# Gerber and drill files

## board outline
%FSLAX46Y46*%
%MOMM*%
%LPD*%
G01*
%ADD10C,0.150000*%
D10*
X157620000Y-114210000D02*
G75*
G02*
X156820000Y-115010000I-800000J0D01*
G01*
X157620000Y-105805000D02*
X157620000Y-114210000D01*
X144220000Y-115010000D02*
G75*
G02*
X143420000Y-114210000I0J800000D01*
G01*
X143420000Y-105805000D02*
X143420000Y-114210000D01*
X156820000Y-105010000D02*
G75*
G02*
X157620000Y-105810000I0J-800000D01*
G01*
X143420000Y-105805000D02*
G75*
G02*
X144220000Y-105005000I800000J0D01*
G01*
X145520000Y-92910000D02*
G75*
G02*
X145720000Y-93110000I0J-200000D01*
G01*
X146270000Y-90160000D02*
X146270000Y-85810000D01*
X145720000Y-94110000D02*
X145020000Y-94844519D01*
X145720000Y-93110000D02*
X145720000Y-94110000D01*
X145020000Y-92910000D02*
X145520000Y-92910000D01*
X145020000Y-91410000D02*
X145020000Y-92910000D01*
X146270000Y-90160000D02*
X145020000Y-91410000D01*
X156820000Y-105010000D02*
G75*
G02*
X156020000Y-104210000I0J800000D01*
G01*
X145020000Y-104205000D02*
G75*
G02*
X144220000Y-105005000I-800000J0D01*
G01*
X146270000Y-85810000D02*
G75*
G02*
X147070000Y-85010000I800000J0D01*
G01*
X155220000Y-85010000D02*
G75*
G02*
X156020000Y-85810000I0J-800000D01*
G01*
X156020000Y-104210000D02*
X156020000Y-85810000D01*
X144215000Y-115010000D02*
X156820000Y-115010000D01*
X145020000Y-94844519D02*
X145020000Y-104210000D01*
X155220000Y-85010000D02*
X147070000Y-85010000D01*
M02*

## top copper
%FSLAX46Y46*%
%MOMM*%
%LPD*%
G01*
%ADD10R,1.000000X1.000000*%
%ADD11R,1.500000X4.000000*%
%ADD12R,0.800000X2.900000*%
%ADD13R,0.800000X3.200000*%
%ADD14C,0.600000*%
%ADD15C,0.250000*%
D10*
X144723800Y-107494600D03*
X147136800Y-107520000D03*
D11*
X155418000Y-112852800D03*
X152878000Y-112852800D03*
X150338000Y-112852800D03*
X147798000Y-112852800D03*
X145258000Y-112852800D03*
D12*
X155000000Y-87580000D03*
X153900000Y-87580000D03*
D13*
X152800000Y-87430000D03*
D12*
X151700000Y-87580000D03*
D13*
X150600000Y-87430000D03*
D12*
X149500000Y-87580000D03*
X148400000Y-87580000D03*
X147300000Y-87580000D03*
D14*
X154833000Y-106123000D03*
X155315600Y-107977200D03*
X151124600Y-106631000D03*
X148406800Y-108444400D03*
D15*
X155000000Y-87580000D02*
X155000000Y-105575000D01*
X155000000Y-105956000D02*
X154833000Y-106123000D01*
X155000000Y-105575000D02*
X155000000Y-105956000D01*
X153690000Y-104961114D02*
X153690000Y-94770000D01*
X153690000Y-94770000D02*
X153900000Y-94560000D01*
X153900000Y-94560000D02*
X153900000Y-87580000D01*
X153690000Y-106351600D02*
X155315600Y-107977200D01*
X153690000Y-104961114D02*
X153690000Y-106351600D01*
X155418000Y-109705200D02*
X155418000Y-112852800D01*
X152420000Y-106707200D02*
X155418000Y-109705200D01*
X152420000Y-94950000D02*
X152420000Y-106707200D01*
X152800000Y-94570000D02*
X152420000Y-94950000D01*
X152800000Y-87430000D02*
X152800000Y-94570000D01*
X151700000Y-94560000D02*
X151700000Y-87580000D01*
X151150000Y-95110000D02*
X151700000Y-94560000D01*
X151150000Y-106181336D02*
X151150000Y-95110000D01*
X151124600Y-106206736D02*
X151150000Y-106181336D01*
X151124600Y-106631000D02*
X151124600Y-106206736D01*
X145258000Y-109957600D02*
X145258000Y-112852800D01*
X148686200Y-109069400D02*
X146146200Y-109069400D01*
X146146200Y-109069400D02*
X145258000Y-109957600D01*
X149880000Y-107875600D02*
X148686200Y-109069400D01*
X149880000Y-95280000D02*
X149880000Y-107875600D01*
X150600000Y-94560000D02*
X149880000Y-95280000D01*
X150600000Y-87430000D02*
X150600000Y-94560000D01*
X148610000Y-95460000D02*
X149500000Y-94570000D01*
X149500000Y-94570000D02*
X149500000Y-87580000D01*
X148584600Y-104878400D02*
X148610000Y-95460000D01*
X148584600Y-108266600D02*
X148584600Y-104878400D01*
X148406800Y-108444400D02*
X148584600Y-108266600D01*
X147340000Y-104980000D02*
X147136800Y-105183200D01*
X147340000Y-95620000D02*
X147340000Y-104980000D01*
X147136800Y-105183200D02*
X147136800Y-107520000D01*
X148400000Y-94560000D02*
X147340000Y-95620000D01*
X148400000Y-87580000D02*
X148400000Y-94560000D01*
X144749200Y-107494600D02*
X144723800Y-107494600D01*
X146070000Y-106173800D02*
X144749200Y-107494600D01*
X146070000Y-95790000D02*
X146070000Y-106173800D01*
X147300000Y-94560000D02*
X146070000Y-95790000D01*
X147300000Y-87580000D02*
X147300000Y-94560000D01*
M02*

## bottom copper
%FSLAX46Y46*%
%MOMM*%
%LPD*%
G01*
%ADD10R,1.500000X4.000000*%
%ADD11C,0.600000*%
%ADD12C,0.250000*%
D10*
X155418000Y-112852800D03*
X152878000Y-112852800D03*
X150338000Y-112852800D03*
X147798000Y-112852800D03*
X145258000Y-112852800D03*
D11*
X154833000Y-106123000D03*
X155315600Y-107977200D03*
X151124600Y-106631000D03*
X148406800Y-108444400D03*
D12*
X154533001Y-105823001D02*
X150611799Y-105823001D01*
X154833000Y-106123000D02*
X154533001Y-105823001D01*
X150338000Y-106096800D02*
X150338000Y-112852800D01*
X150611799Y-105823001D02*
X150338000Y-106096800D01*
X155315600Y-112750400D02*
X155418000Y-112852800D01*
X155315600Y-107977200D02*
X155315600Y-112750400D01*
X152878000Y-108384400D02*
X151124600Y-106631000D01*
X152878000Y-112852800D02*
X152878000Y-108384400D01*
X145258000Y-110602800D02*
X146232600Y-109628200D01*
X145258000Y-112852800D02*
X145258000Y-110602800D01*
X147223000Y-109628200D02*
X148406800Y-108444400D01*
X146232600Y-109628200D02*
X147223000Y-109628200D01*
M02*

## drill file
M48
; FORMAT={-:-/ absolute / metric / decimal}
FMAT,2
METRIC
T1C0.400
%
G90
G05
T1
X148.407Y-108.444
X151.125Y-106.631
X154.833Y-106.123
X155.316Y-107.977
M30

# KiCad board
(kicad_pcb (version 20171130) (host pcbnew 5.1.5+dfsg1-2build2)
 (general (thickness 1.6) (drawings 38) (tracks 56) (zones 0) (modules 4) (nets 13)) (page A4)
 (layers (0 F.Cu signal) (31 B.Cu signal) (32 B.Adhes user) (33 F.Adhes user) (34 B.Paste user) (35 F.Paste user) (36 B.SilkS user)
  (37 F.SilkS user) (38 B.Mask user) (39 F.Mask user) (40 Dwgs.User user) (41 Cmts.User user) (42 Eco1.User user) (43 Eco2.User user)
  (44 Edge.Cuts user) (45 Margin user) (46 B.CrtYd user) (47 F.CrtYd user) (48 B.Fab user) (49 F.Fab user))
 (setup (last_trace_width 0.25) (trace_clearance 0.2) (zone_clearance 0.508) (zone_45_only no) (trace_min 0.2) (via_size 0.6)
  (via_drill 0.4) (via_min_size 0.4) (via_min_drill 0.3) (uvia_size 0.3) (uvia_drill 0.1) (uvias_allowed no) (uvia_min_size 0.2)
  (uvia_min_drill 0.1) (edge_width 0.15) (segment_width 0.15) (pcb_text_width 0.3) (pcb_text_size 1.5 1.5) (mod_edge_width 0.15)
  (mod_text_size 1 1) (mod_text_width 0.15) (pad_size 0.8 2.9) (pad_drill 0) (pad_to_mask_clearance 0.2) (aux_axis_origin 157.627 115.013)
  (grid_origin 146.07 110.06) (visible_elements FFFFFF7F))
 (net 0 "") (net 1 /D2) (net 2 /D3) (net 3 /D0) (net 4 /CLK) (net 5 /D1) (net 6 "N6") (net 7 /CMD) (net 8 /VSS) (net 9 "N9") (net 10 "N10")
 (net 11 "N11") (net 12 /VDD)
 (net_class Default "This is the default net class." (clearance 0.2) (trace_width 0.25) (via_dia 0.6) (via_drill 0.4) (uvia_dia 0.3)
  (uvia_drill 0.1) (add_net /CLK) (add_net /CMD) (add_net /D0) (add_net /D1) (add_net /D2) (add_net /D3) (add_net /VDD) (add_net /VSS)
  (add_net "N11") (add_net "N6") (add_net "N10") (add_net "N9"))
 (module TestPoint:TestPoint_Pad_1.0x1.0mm (layer F.Cu) (at 144.7238 107.4946)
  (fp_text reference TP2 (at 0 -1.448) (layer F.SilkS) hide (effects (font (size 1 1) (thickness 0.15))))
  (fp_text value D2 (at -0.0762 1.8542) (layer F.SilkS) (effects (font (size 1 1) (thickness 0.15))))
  (pad 1 smd rect (at 0 0) (size 1 1) (layers F.Cu F.Mask) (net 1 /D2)))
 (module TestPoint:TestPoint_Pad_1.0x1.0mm (layer F.Cu) (at 147.1368 107.52 90)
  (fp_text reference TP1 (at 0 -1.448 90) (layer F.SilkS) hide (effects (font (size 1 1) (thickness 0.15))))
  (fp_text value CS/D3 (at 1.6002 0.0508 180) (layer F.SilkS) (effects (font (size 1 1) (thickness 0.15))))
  (pad 1 smd rect (at 0 0 90) (size 1 1) (layers F.Cu F.Mask) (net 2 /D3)))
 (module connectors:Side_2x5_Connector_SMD (layer F.Cu) (at 150.388 112.7778 270)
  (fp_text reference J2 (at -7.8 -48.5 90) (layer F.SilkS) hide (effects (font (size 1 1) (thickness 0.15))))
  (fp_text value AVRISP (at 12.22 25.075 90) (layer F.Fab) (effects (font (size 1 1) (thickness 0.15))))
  (pad 10 smd rect (at 0.075 -5.03 270) (size 4 1.5) (layers B.Cu B.Paste B.Mask) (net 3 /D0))
  (pad 8 smd rect (at 0.075 -2.49 270) (size 4 1.5) (layers B.Cu B.Paste B.Mask) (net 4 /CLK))
  (pad 6 smd rect (at 0.075 0.05 270) (size 4 1.5) (layers B.Cu B.Paste B.Mask) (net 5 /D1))
  (pad 4 smd rect (at 0.075 2.59 270) (size 4 1.5) (layers B.Cu B.Paste B.Mask) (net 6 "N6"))
  (pad 2 smd rect (at 0.075 5.13 270) (size 4 1.5) (layers B.Cu B.Paste B.Mask) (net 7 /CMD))
  (pad 9 smd rect (at 0.075 -5.03 270) (size 4 1.5) (layers F.Cu F.Paste F.Mask) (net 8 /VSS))
  (pad 7 smd rect (at 0.075 -2.49 270) (size 4 1.5) (layers F.Cu F.Paste F.Mask) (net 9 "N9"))
  (pad 5 smd rect (at 0.075 0.05 270) (size 4 1.5) (layers F.Cu F.Paste F.Mask) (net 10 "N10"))
  (pad 3 smd rect (at 0.075 2.59 270) (size 4 1.5) (layers F.Cu F.Paste F.Mask) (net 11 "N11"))
  (pad 1 smd rect (at 0.075 5.13 270) (size 4 1.5) (layers F.Cu F.Paste F.Mask) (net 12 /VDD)))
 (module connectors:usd (layer F.Cu) (at 147.3 87.58)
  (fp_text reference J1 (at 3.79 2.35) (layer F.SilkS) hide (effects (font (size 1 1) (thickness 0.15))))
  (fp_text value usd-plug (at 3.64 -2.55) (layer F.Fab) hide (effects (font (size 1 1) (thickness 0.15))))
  (pad 8 smd rect (at 7.7 0) (size 0.8 2.9) (layers F.Cu F.Paste F.Mask) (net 5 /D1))
  (pad 7 smd rect (at 6.6 0) (size 0.8 2.9) (layers F.Cu F.Paste F.Mask) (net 3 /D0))
  (pad 6 smd rect (at 5.5 -0.15) (size 0.8 3.2) (layers F.Cu F.Paste F.Mask) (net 8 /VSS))
  (pad 5 smd rect (at 4.4 0) (size 0.8 2.9) (layers F.Cu F.Paste F.Mask) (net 4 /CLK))
  (pad 4 smd rect (at 3.3 -0.15) (size 0.8 3.2) (layers F.Cu F.Paste F.Mask) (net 12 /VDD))
  (pad 3 smd rect (at 2.2 0) (size 0.8 2.9) (layers F.Cu F.Paste F.Mask) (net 7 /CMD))
  (pad 2 smd rect (at 1.1 0) (size 0.8 2.9) (layers F.Cu F.Paste F.Mask) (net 2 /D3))
  (pad 1 smd rect (at 0 0) (size 0.8 2.9) (layers F.Cu F.Paste F.Mask) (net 1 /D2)))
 (gr_arc (start 156.82 114.21) (end 157.62 114.21) (angle 90) (layer Edge.Cuts) (width 0.15))
 (gr_line (start 157.62 105.805) (end 157.62 114.21) (angle 90) (layer Edge.Cuts) (width 0.15))
 (gr_arc (start 144.22 114.21) (end 144.22 115.01) (angle 90) (layer Edge.Cuts) (width 0.15))
 (gr_line (start 143.42 105.805) (end 143.42 114.21) (angle 90) (layer Edge.Cuts) (width 0.15))
 (gr_arc (start 156.82 105.81) (end 156.82 105.01) (angle 90) (layer Edge.Cuts) (width 0.15))
 (gr_arc (start 144.22 105.805) (end 143.42 105.805) (angle 90) (layer Edge.Cuts) (width 0.15))
 (gr_arc (start 145.52 93.11) (end 145.72 93.11) (angle -90) (layer Edge.Cuts) (width 0.15))
 (gr_line (start 146.27 90.16) (end 146.27 85.81) (angle 90) (layer Edge.Cuts) (width 0.15))
 (gr_line (start 145.72 94.11) (end 145.02 94.844519) (angle 90) (layer Edge.Cuts) (width 0.15))
 (gr_line (start 145.72 93.11) (end 145.72 94.11) (angle 90) (layer Edge.Cuts) (width 0.15))
 (gr_line (start 145.02 92.91) (end 145.52 92.91) (angle 90) (layer Edge.Cuts) (width 0.15))
 (gr_line (start 145.02 91.41) (end 145.02 92.91) (angle 90) (layer Edge.Cuts) (width 0.15))
 (gr_line (start 146.27 90.16) (end 145.02 91.41) (angle 90) (layer Edge.Cuts) (width 0.15))
 (gr_arc (start 156.82 104.21) (end 156.82 105.01) (angle 90) (layer Edge.Cuts) (width 0.15))
 (gr_arc (start 144.22 104.205) (end 145.02 104.205) (angle 90) (layer Edge.Cuts) (width 0.15))
 (gr_arc (start 147.07 85.81) (end 147.07 85.01) (angle -90) (layer Edge.Cuts) (width 0.15))
 (gr_arc (start 155.22 85.81) (end 156.02 85.81) (angle -90) (layer Edge.Cuts) (width 0.15))
 (gr_line (start 156.02 104.21) (end 156.02 85.81) (angle 90) (layer Edge.Cuts) (width 0.15))
 (gr_line (start 144.215 115.01) (end 156.82 115.01) (angle 90) (layer Edge.Cuts) (width 0.15))
 (gr_line (start 145.02 94.844519) (end 145.02 104.21) (angle 90) (layer Edge.Cuts) (width 0.15))
 (gr_line (start 155.22 85.01) (end 147.07 85.01) (angle 90) (layer Edge.Cuts) (width 0.15))
 (segment (start 155 87.58) (end 155 105.575) (width 0.25) (layer F.Cu) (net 5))
 (via (at 154.833 106.123) (size 0.6) (drill 0.4) (layers F.Cu B.Cu) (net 5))
 (segment (start 155 105.956) (end 154.833 106.123) (width 0.25) (layer F.Cu) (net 5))
 (segment (start 155 105.575) (end 155 105.956) (width 0.25) (layer F.Cu) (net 5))
 (segment (start 154.533001 105.823001) (end 150.611799 105.823001) (width 0.25) (layer B.Cu) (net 5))
 (segment (start 154.833 106.123) (end 154.533001 105.823001) (width 0.25) (layer B.Cu) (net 5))
 (segment (start 150.338 106.0968) (end 150.338 112.8528) (width 0.25) (layer B.Cu) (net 5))
 (segment (start 150.611799 105.823001) (end 150.338 106.0968) (width 0.25) (layer B.Cu) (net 5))
 (segment (start 153.69 104.961114) (end 153.69 94.77) (width 0.25) (layer F.Cu) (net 3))
 (segment (start 153.69 94.77) (end 153.9 94.56) (width 0.25) (layer F.Cu) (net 3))
 (segment (start 153.9 94.56) (end 153.9 87.58) (width 0.25) (layer F.Cu) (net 3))
 (via (at 155.3156 107.9772) (size 0.6) (drill 0.4) (layers F.Cu B.Cu) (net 3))
 (segment (start 153.69 106.3516) (end 155.3156 107.9772) (width 0.25) (layer F.Cu) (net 3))
 (segment (start 153.69 104.961114) (end 153.69 106.3516) (width 0.25) (layer F.Cu) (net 3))
 (segment (start 155.3156 112.7504) (end 155.418 112.8528) (width 0.25) (layer B.Cu) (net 3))
 (segment (start 155.3156 107.9772) (end 155.3156 112.7504) (width 0.25) (layer B.Cu) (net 3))
 (segment (start 155.418 109.7052) (end 155.418 112.8528) (width 0.25) (layer F.Cu) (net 8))
 (segment (start 152.42 106.7072) (end 155.418 109.7052) (width 0.25) (layer F.Cu) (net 8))
 (segment (start 152.42 94.95) (end 152.42 106.7072) (width 0.25) (layer F.Cu) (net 8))
 (segment (start 152.8 94.57) (end 152.42 94.95) (width 0.25) (layer F.Cu) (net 8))
 (segment (start 152.8 87.43) (end 152.8 94.57) (width 0.25) (layer F.Cu) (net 8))
 (via (at 151.1246 106.631) (size 0.6) (drill 0.4) (layers F.Cu B.Cu) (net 4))
 (segment (start 152.878 108.3844) (end 151.1246 106.631) (width 0.25) (layer B.Cu) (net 4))
 (segment (start 152.878 112.8528) (end 152.878 108.3844) (width 0.25) (layer B.Cu) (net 4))
 (segment (start 151.7 94.56) (end 151.7 87.58) (width 0.25) (layer F.Cu) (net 4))
 (segment (start 151.15 95.11) (end 151.7 94.56) (width 0.25) (layer F.Cu) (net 4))
 (segment (start 151.15 106.181336) (end 151.15 95.11) (width 0.25) (layer F.Cu) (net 4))
 (segment (start 151.1246 106.206736) (end 151.15 106.181336) (width 0.25) (layer F.Cu) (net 4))
 (segment (start 151.1246 106.631) (end 151.1246 106.206736) (width 0.25) (layer F.Cu) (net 4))
 (segment (start 145.258 109.9576) (end 145.258 112.8528) (width 0.25) (layer F.Cu) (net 12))
 (segment (start 148.6862 109.0694) (end 146.1462 109.0694) (width 0.25) (layer F.Cu) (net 12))
 (segment (start 146.1462 109.0694) (end 145.258 109.9576) (width 0.25) (layer F.Cu) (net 12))
 (segment (start 149.88 107.8756) (end 148.6862 109.0694) (width 0.25) (layer F.Cu) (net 12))
 (segment (start 149.88 95.28) (end 149.88 107.8756) (width 0.25) (layer F.Cu) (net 12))
 (segment (start 150.6 94.56) (end 149.88 95.28) (width 0.25) (layer F.Cu) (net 12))
 (segment (start 150.6 87.43) (end 150.6 94.56) (width 0.25) (layer F.Cu) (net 12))
 (segment (start 148.61 95.46) (end 149.5 94.57) (width 0.25) (layer F.Cu) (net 7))
 (segment (start 149.5 94.57) (end 149.5 87.58) (width 0.25) (layer F.Cu) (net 7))
 (segment (start 145.258 110.6028) (end 146.2326 109.6282) (width 0.25) (layer B.Cu) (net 7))
 (segment (start 145.258 112.8528) (end 145.258 110.6028) (width 0.25) (layer B.Cu) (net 7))
 (via (at 148.4068 108.4444) (size 0.6) (drill 0.4) (layers F.Cu B.Cu) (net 7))
 (segment (start 147.223 109.6282) (end 148.4068 108.4444) (width 0.25) (layer B.Cu) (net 7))
 (segment (start 146.2326 109.6282) (end 147.223 109.6282) (width 0.25) (layer B.Cu) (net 7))
 (segment (start 148.5846 104.8784) (end 148.61 95.46) (width 0.25) (layer F.Cu) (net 7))
 (segment (start 148.5846 108.2666) (end 148.5846 104.8784) (width 0.25) (layer F.Cu) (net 7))
 (segment (start 148.4068 108.4444) (end 148.5846 108.2666) (width 0.25) (layer F.Cu) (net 7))
 (segment (start 147.34 104.98) (end 147.1368 105.1832) (width 0.25) (layer F.Cu) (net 2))
 (segment (start 147.34 95.62) (end 147.34 104.98) (width 0.25) (layer F.Cu) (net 2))
 (segment (start 147.1368 105.1832) (end 147.1368 107.52) (width 0.25) (layer F.Cu) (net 2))
 (segment (start 148.4 94.56) (end 147.34 95.62) (width 0.25) (layer F.Cu) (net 2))
 (segment (start 148.4 87.58) (end 148.4 94.56) (width 0.25) (layer F.Cu) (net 2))
 (segment (start 144.7492 107.4946) (end 144.7238 107.4946) (width 0.25) (layer F.Cu) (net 1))
 (segment (start 146.07 106.1738) (end 144.7492 107.4946) (width 0.25) (layer F.Cu) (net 1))
 (segment (start 146.07 95.79) (end 146.07 106.1738) (width 0.25) (layer F.Cu) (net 1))
 (segment (start 147.3 94.56) (end 146.07 95.79) (width 0.25) (layer F.Cu) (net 1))
 (segment (start 147.3 87.58) (end 147.3 94.56) (width 0.25) (layer F.Cu) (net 1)))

